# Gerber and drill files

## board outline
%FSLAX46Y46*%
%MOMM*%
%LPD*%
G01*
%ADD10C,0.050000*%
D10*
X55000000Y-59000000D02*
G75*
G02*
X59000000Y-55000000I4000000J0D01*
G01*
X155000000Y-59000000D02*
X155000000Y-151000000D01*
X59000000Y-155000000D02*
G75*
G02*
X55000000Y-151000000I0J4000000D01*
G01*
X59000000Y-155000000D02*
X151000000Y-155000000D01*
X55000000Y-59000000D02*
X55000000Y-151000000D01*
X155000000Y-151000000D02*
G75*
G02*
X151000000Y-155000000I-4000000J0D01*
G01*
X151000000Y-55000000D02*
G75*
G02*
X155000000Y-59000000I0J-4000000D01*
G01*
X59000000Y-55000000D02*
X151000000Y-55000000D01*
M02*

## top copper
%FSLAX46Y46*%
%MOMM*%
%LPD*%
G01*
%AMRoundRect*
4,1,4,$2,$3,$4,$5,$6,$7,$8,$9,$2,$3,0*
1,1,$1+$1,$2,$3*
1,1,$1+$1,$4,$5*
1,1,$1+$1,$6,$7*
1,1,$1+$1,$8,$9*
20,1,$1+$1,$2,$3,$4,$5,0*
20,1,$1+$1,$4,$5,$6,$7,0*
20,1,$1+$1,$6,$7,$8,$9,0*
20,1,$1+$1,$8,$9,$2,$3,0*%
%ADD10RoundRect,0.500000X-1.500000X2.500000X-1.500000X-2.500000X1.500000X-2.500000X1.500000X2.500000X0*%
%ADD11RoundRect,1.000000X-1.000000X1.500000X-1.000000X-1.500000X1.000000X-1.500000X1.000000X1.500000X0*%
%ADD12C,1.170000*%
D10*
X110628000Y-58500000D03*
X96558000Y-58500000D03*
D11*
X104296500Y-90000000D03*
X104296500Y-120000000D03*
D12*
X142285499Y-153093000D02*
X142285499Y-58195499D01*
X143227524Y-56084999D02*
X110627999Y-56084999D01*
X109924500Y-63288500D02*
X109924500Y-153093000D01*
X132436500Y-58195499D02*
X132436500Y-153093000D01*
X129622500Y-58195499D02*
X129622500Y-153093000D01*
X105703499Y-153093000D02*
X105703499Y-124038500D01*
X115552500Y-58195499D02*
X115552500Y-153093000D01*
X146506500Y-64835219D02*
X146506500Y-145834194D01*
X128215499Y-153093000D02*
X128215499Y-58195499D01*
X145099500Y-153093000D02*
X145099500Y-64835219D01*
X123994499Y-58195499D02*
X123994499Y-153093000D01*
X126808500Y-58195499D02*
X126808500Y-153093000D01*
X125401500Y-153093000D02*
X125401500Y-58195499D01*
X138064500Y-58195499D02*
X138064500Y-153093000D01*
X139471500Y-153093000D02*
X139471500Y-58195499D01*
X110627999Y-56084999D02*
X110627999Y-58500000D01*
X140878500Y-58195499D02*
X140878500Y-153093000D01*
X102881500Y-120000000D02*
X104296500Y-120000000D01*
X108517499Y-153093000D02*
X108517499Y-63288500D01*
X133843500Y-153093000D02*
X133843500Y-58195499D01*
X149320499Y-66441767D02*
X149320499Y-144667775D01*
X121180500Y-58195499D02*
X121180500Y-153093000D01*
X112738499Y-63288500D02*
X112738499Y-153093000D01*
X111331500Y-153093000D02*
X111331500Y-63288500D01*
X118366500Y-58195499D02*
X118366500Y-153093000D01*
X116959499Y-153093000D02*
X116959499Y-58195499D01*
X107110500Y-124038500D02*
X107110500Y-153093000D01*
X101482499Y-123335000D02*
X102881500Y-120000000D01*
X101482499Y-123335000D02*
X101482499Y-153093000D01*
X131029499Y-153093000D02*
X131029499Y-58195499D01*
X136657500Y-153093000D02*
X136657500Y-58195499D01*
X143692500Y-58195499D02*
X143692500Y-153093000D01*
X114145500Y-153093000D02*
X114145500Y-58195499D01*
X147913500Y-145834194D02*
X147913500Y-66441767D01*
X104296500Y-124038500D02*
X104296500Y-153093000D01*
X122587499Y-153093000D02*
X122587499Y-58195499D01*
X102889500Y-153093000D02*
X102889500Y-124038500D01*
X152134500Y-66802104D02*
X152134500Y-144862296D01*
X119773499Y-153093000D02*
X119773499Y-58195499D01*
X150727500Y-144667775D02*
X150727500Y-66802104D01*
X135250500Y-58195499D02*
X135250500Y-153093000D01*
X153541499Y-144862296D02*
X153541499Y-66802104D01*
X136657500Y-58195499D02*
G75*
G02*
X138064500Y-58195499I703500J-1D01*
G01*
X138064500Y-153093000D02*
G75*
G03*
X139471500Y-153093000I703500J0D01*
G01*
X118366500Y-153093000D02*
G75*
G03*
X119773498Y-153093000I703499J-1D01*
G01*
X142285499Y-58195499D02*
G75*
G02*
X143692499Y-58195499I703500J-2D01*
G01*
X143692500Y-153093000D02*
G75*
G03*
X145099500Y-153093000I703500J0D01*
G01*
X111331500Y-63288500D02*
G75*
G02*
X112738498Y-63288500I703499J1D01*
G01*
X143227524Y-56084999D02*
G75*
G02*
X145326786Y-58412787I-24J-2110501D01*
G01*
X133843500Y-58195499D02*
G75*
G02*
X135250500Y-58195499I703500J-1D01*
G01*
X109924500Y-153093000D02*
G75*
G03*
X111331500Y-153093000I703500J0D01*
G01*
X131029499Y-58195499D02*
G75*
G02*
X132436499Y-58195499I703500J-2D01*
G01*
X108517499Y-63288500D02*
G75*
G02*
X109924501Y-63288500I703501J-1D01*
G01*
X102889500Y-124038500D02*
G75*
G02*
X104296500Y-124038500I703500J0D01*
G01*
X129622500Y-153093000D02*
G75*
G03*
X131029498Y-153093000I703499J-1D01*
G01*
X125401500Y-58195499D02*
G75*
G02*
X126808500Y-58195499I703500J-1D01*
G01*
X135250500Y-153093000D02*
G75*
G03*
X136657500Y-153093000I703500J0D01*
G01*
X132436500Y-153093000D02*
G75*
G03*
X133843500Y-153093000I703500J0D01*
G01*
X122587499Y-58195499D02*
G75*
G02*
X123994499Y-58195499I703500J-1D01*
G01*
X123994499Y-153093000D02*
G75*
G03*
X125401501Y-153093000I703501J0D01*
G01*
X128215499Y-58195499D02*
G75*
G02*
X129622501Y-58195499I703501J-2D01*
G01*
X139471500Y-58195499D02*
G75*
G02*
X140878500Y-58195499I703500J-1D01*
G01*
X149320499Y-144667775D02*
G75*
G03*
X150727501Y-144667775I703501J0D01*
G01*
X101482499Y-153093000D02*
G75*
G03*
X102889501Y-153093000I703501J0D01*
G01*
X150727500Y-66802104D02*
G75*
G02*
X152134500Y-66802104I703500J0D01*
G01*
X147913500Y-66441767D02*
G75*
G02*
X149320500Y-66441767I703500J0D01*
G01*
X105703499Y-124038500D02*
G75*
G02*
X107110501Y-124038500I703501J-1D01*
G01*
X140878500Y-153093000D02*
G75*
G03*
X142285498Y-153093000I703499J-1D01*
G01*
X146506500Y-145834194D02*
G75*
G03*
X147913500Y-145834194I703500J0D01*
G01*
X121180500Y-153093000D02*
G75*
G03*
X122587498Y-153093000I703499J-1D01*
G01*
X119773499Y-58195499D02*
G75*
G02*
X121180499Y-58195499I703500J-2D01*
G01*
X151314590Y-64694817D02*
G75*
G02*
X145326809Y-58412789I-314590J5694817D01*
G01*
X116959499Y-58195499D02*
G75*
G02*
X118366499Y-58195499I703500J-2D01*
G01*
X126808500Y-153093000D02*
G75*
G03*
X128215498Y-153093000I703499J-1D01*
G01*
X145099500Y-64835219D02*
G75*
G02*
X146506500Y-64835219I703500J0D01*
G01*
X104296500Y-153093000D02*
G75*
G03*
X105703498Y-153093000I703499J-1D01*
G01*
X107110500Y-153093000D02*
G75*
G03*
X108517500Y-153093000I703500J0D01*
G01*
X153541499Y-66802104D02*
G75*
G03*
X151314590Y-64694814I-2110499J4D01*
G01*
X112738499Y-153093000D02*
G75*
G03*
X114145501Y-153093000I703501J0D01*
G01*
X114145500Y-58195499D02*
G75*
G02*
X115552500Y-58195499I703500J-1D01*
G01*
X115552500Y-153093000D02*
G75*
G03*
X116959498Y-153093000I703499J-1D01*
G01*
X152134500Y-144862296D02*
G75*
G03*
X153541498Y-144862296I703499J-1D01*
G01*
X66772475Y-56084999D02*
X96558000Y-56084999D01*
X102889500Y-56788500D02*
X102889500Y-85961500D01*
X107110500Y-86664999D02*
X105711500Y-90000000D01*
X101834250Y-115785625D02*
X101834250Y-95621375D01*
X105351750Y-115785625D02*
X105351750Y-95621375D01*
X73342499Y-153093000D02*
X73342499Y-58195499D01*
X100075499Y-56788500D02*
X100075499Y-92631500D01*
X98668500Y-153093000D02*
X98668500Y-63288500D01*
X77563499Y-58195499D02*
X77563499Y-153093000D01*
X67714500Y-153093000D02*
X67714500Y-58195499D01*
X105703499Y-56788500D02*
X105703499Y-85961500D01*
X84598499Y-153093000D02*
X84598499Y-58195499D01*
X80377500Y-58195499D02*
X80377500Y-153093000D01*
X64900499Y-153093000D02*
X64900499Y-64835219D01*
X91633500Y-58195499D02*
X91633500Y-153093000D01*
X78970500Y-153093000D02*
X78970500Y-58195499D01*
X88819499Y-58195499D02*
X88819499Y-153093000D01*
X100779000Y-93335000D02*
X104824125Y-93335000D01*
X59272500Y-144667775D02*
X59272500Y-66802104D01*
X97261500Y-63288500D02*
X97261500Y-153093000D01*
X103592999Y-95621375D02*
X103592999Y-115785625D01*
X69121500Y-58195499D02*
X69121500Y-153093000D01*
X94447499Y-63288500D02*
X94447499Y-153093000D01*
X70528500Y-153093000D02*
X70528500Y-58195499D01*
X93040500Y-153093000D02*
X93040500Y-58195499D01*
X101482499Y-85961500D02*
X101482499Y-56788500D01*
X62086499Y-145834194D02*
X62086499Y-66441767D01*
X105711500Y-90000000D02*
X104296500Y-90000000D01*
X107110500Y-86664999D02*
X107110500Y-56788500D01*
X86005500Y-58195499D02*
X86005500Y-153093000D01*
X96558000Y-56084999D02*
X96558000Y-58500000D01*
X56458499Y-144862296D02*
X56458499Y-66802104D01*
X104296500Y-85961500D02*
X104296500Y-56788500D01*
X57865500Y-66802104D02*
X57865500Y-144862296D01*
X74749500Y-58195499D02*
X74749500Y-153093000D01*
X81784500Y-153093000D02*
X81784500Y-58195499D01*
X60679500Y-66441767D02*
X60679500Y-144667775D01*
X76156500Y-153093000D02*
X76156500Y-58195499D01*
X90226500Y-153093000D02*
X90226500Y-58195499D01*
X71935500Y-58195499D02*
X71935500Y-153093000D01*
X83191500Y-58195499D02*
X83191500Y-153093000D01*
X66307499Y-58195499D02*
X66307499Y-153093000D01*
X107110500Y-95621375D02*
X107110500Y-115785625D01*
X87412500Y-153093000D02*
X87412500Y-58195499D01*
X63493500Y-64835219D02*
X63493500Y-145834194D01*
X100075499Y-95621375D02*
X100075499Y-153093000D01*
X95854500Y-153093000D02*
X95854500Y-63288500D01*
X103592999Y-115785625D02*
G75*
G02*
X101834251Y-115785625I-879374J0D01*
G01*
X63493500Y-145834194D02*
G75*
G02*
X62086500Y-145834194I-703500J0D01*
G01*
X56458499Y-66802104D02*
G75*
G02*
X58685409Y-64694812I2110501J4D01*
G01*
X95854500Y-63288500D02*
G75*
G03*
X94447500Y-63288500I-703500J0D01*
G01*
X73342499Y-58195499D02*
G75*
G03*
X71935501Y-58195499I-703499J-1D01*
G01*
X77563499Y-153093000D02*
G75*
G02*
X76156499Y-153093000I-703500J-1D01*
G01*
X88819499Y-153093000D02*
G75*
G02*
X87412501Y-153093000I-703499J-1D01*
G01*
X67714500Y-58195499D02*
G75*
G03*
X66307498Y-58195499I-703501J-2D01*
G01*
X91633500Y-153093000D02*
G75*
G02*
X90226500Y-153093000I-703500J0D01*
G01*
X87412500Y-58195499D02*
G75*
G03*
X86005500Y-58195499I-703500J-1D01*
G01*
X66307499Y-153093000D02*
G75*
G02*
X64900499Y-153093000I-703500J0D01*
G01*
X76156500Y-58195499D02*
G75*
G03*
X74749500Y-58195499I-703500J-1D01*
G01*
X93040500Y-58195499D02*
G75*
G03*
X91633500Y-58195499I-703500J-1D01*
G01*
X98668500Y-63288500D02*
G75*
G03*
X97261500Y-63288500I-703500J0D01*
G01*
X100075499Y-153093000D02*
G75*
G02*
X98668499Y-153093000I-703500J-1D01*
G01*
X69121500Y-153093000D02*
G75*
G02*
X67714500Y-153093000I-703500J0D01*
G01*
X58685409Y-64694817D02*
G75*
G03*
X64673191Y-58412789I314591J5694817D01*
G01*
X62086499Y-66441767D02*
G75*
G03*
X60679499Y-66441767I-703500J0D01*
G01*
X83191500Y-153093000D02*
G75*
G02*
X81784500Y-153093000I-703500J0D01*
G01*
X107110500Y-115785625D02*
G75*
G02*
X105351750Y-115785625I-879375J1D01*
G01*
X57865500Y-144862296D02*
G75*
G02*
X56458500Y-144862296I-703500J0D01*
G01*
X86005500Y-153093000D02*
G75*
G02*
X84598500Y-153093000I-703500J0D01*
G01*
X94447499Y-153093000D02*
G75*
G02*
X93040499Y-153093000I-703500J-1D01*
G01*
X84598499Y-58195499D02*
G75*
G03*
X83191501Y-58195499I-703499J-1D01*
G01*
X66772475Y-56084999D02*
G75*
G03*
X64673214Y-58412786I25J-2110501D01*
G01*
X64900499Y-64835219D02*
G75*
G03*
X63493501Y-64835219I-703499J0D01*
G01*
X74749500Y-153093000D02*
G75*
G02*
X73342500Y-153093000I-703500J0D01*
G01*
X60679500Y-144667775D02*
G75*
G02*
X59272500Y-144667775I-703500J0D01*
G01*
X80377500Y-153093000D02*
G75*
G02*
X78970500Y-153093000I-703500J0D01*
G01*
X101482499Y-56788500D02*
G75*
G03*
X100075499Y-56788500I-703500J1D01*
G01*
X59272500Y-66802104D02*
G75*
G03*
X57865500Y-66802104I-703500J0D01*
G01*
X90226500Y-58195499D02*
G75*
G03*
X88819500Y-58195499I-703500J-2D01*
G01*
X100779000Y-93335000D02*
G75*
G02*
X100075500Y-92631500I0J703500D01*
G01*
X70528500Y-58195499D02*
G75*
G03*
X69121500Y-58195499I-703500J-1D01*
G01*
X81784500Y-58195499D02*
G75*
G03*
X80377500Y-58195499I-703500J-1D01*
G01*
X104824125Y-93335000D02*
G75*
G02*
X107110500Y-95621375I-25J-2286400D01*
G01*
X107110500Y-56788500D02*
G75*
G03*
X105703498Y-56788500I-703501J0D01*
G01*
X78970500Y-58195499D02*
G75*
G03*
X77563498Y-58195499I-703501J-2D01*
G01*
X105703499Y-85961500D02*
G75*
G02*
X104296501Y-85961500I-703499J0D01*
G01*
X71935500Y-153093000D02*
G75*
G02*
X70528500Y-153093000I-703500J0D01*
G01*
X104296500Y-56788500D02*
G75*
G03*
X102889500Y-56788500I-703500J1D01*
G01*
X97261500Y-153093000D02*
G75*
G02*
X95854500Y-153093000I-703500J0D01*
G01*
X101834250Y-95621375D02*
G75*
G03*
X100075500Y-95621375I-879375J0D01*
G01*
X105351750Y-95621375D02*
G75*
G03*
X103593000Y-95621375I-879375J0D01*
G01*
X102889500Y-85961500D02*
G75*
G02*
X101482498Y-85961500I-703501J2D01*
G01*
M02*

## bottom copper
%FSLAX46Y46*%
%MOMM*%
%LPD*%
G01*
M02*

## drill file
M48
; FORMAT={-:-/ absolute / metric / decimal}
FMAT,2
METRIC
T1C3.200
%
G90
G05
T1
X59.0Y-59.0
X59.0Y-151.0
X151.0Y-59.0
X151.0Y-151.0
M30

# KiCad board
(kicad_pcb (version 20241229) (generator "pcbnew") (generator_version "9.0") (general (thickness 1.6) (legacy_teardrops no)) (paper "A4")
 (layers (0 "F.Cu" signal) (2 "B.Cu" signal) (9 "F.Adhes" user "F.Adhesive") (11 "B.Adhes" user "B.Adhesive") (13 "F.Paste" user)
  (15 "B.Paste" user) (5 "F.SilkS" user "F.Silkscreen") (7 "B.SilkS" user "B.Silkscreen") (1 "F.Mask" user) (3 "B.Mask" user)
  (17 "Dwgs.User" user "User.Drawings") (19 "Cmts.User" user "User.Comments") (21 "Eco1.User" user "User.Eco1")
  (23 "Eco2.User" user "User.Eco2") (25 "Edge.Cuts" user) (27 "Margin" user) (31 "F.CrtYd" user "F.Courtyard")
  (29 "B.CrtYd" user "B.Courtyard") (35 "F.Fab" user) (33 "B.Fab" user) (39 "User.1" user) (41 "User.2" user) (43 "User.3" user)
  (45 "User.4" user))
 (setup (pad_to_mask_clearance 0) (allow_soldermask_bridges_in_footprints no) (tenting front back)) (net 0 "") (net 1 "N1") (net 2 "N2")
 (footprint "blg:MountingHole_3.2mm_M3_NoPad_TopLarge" (layer "F.Cu") (at 151 59)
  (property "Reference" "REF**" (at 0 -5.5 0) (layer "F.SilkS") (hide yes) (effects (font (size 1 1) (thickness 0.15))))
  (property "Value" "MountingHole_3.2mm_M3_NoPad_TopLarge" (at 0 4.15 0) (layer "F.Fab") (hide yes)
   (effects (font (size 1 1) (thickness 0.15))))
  (pad "" np_thru_hole circle (at 0 0) (size 7.6 7.6) (drill 3.2) (layers) (zone_connect 2)))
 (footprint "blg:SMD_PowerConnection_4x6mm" (layer "F.Cu") (at 110.628 58.5 -90)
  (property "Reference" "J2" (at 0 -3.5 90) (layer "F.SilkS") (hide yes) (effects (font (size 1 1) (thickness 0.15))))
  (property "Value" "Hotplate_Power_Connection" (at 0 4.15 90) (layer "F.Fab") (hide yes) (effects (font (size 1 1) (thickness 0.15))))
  (pad "1" smd roundrect (at 0 0 270) (size 6 4) (layers "F.Cu" "F.Mask" "F.Paste") (roundrect_rratio 0.125) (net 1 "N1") (zone_connect 2)))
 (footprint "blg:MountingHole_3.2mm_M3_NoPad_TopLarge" (layer "F.Cu") (at 59 151)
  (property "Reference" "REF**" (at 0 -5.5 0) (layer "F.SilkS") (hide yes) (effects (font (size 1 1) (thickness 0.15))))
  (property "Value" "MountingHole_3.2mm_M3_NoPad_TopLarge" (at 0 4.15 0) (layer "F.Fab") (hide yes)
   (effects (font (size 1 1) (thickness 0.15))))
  (pad "" np_thru_hole circle (at 0 0) (size 7.6 7.6) (drill 3.2) (layers) (zone_connect 2)))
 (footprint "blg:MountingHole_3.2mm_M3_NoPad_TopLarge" (layer "F.Cu") (at 151 151)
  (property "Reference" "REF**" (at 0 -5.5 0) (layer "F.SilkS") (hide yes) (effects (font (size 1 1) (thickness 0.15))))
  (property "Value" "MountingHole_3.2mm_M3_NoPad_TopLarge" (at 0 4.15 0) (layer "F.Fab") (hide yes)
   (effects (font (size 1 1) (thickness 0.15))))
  (pad "" np_thru_hole circle (at 0 0) (size 7.6 7.6) (drill 3.2) (layers) (zone_connect 2)))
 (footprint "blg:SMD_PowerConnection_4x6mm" (layer "F.Cu") (at 96.558 58.5 -90)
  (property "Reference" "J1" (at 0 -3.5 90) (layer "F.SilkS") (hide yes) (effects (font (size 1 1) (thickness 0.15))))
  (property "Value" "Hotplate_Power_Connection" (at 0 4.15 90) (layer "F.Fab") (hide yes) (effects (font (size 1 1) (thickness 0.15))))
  (pad "1" smd roundrect (at 0 0 270) (size 6 4) (layers "F.Cu" "F.Mask" "F.Paste") (roundrect_rratio 0.125) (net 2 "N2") (zone_connect 2)))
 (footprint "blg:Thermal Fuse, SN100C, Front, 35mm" (layer "F.Cu") (at 104.2965 105 -90)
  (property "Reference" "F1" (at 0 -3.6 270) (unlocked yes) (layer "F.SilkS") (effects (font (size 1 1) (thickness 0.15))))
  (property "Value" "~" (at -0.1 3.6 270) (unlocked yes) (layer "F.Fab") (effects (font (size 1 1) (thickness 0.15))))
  (pad "1" smd roundrect (at -15 0 270) (size 5 4) (layers "F.Cu" "F.Mask") (roundrect_rratio 0.25) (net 2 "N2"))
  (pad "2" smd roundrect (at 15 0 270) (size 5 4) (layers "F.Cu" "F.Mask") (roundrect_rratio 0.25) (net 1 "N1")))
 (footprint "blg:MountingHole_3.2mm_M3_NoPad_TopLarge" (layer "F.Cu") (at 59 59)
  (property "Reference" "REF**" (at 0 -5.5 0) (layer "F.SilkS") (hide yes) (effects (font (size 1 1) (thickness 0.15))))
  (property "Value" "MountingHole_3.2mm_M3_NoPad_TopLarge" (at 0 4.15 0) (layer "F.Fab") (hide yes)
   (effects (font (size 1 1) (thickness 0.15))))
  (pad "" np_thru_hole circle (at 0 0) (size 7.6 7.6) (drill 3.2) (layers) (zone_connect 2)))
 (gr_arc (start 55 59) (mid 56.171573 56.171573) (end 59 55) (stroke (width 0.05) (type solid)) (layer "Edge.Cuts"))
 (gr_line (start 155 59) (end 155 151) (stroke (width 0.05) (type default)) (layer "Edge.Cuts"))
 (gr_arc (start 59 155) (mid 56.171573 153.828427) (end 55 151) (stroke (width 0.05) (type solid)) (layer "Edge.Cuts"))
 (gr_line (start 59 155) (end 151 155) (stroke (width 0.05) (type default)) (layer "Edge.Cuts"))
 (gr_line (start 55 59) (end 55 151) (stroke (width 0.05) (type default)) (layer "Edge.Cuts"))
 (gr_arc (start 155 151) (mid 153.828427 153.828427) (end 151 155) (stroke (width 0.05) (type solid)) (layer "Edge.Cuts"))
 (gr_arc (start 151 55) (mid 153.828427 56.171573) (end 155 59) (stroke (width 0.05) (type solid)) (layer "Edge.Cuts"))
 (gr_line (start 59 55) (end 151 55) (stroke (width 0.05) (type default)) (layer "Edge.Cuts"))
 (segment (start 142.285499 153.093) (end 142.285499 58.195499) (width 1.17) (layer "F.Cu") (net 1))
 (segment (start 143.227524 56.084999) (end 110.627999 56.084999) (width 1.17) (layer "F.Cu") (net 1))
 (segment (start 109.9245 63.2885) (end 109.9245 153.093) (width 1.17) (layer "F.Cu") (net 1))
 (segment (start 132.4365 58.195499) (end 132.4365 153.093) (width 1.17) (layer "F.Cu") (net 1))
 (segment (start 129.6225 58.195499) (end 129.6225 153.093) (width 1.17) (layer "F.Cu") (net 1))
 (segment (start 105.703499 153.093) (end 105.703499 124.0385) (width 1.17) (layer "F.Cu") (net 1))
 (segment (start 115.5525 58.195499) (end 115.5525 153.093) (width 1.17) (layer "F.Cu") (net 1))
 (segment (start 146.5065 64.835219) (end 146.5065 145.834194) (width 1.17) (layer "F.Cu") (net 1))
 (segment (start 128.215499 153.093) (end 128.215499 58.195499) (width 1.17) (layer "F.Cu") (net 1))
 (segment (start 145.0995 153.093) (end 145.0995 64.835219) (width 1.17) (layer "F.Cu") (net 1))
 (segment (start 123.994499 58.195499) (end 123.994499 153.093) (width 1.17) (layer "F.Cu") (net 1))
 (segment (start 126.8085 58.195499) (end 126.8085 153.093) (width 1.17) (layer "F.Cu") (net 1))
 (segment (start 125.4015 153.093) (end 125.4015 58.195499) (width 1.17) (layer "F.Cu") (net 1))
 (segment (start 138.0645 58.195499) (end 138.0645 153.093) (width 1.17) (layer "F.Cu") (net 1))
 (segment (start 139.4715 153.093) (end 139.4715 58.195499) (width 1.17) (layer "F.Cu") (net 1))
 (segment (start 110.627999 56.084999) (end 110.627999 58.5) (width 1.17) (layer "F.Cu") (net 1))
 (segment (start 140.8785 58.195499) (end 140.8785 153.093) (width 1.17) (layer "F.Cu") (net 1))
 (segment (start 102.8815 120) (end 104.2965 120) (width 1.17) (layer "F.Cu") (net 1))
 (segment (start 108.517499 153.093) (end 108.517499 63.2885) (width 1.17) (layer "F.Cu") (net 1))
 (segment (start 133.8435 153.093) (end 133.8435 58.195499) (width 1.17) (layer "F.Cu") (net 1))
 (segment (start 149.320499 66.441767) (end 149.320499 144.667775) (width 1.17) (layer "F.Cu") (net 1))
 (segment (start 121.1805 58.195499) (end 121.1805 153.093) (width 1.17) (layer "F.Cu") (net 1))
 (segment (start 112.738499 63.2885) (end 112.738499 153.093) (width 1.17) (layer "F.Cu") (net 1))
 (segment (start 111.3315 153.093) (end 111.3315 63.2885) (width 1.17) (layer "F.Cu") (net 1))
 (segment (start 118.3665 58.195499) (end 118.3665 153.093) (width 1.17) (layer "F.Cu") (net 1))
 (segment (start 116.959499 153.093) (end 116.959499 58.195499) (width 1.17) (layer "F.Cu") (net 1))
 (segment (start 107.1105 124.0385) (end 107.1105 153.093) (width 1.17) (layer "F.Cu") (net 1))
 (segment (start 101.482499 123.335) (end 102.8815 120) (width 1.17) (layer "F.Cu") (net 1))
 (segment (start 101.482499 123.335) (end 101.482499 153.093) (width 1.17) (layer "F.Cu") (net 1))
 (segment (start 131.029499 153.093) (end 131.029499 58.195499) (width 1.17) (layer "F.Cu") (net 1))
 (segment (start 136.6575 153.093) (end 136.6575 58.195499) (width 1.17) (layer "F.Cu") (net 1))
 (segment (start 143.6925 58.195499) (end 143.6925 153.093) (width 1.17) (layer "F.Cu") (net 1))
 (segment (start 114.1455 153.093) (end 114.1455 58.195499) (width 1.17) (layer "F.Cu") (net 1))
 (segment (start 147.9135 145.834194) (end 147.9135 66.441767) (width 1.17) (layer "F.Cu") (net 1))
 (segment (start 104.2965 124.0385) (end 104.2965 153.093) (width 1.17) (layer "F.Cu") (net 1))
 (segment (start 122.587499 153.093) (end 122.587499 58.195499) (width 1.17) (layer "F.Cu") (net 1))
 (segment (start 102.8895 153.093) (end 102.8895 124.0385) (width 1.17) (layer "F.Cu") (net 1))
 (segment (start 152.1345 66.802104) (end 152.1345 144.862296) (width 1.17) (layer "F.Cu") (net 1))
 (segment (start 119.773499 153.093) (end 119.773499 58.195499) (width 1.17) (layer "F.Cu") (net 1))
 (segment (start 150.7275 144.667775) (end 150.7275 66.802104) (width 1.17) (layer "F.Cu") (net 1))
 (segment (start 135.2505 58.195499) (end 135.2505 153.093) (width 1.17) (layer "F.Cu") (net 1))
 (segment (start 153.541499 144.862296) (end 153.541499 66.802104) (width 1.17) (layer "F.Cu") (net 1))
 (arc (start 136.6575 58.195499) (mid 137.361 57.492) (end 138.0645 58.195499) (width 1.17) (layer "F.Cu") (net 1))
 (arc (start 138.0645 153.093) (mid 138.768 153.7965) (end 139.4715 153.093) (width 1.17) (layer "F.Cu") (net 1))
 (arc (start 118.3665 153.093) (mid 119.07 153.7965) (end 119.773499 153.093) (width 1.17) (layer "F.Cu") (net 1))
 (arc (start 142.285499 58.195499) (mid 142.989 57.492) (end 143.6925 58.195499) (width 1.17) (layer "F.Cu") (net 1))
 (arc (start 143.6925 153.093) (mid 144.396 153.7965) (end 145.0995 153.093) (width 1.17) (layer "F.Cu") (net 1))
 (arc (start 111.3315 63.2885) (mid 112.035 62.585) (end 112.738499 63.2885) (width 1.17) (layer "F.Cu") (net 1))
 (arc (start 143.227524 56.084999) (mid 144.794814 56.78206) (end 145.326809 58.412789) (width 1.17) (layer "F.Cu") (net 1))
 (arc (start 133.8435 58.195499) (mid 134.547 57.492) (end 135.2505 58.195499) (width 1.17) (layer "F.Cu") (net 1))
 (arc (start 109.9245 153.093) (mid 110.627999 153.7965) (end 111.3315 153.093) (width 1.17) (layer "F.Cu") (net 1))
 (arc (start 131.029499 58.195499) (mid 131.732999 57.492) (end 132.4365 58.195499) (width 1.17) (layer "F.Cu") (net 1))
 (arc (start 108.517499 63.2885) (mid 109.221 62.585) (end 109.9245 63.2885) (width 1.17) (layer "F.Cu") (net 1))
 (arc (start 102.8895 124.0385) (mid 103.592999 123.335) (end 104.2965 124.0385) (width 1.17) (layer "F.Cu") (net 1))
 (arc (start 129.6225 153.093) (mid 130.326 153.7965) (end 131.029499 153.093) (width 1.17) (layer "F.Cu") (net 1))
 (arc (start 125.4015 58.195499) (mid 126.104999 57.492) (end 126.8085 58.195499) (width 1.17) (layer "F.Cu") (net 1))
 (arc (start 135.2505 153.093) (mid 135.953999 153.7965) (end 136.6575 153.093) (width 1.17) (layer "F.Cu") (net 1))
 (arc (start 132.4365 153.093) (mid 133.139999 153.7965) (end 133.8435 153.093) (width 1.17) (layer "F.Cu") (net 1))
 (arc (start 122.587499 58.195499) (mid 123.291 57.492) (end 123.994499 58.195499) (width 1.17) (layer "F.Cu") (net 1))
 (arc (start 123.994499 153.093) (mid 124.698 153.7965) (end 125.4015 153.093) (width 1.17) (layer "F.Cu") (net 1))
 (arc (start 128.215499 58.195499) (mid 128.919 57.492) (end 129.6225 58.195499) (width 1.17) (layer "F.Cu") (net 1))
 (arc (start 139.4715 58.195499) (mid 140.174999 57.492) (end 140.8785 58.195499) (width 1.17) (layer "F.Cu") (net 1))
 (arc (start 149.320499 144.667775) (mid 150.024 145.371275) (end 150.7275 144.667775) (width 1.17) (layer "F.Cu") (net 1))
 (arc (start 101.482499 153.093) (mid 102.186 153.7965) (end 102.8895 153.093) (width 1.17) (layer "F.Cu") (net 1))
 (arc (start 150.7275 66.802104) (mid 151.430999 66.098604) (end 152.1345 66.802104) (width 1.17) (layer "F.Cu") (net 1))
 (arc (start 147.9135 66.441767) (mid 148.617 65.738267) (end 149.320499 66.441767) (width 1.17) (layer "F.Cu") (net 1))
 (arc (start 105.703499 124.0385) (mid 106.407 123.335) (end 107.1105 124.0385) (width 1.17) (layer "F.Cu") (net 1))
 (arc (start 140.8785 153.093) (mid 141.582 153.7965) (end 142.285499 153.093) (width 1.17) (layer "F.Cu") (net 1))
 (arc (start 146.5065 145.834194) (mid 147.209999 146.537694) (end 147.9135 145.834194) (width 1.17) (layer "F.Cu") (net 1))
 (arc (start 121.1805 153.093) (mid 121.883999 153.7965) (end 122.587499 153.093) (width 1.17) (layer "F.Cu") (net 1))
 (arc (start 119.773499 58.195499) (mid 120.477 57.492) (end 121.1805 58.195499) (width 1.17) (layer "F.Cu") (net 1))
 (arc (start 151.31459 64.694817) (mid 146.871486 62.935135) (end 145.326809 58.412789) (width 1.17) (layer "F.Cu") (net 1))
 (arc (start 116.959499 58.195499) (mid 117.663 57.492) (end 118.3665 58.195499) (width 1.17) (layer "F.Cu") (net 1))
 (arc (start 126.8085 153.093) (mid 127.511999 153.7965) (end 128.215499 153.093) (width 1.17) (layer "F.Cu") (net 1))
 (arc (start 145.0995 64.835219) (mid 145.803 64.131719) (end 146.5065 64.835219) (width 1.17) (layer "F.Cu") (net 1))
 (arc (start 104.2965 153.093) (mid 105 153.7965) (end 105.703499 153.093) (width 1.17) (layer "F.Cu") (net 1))
 (arc (start 107.1105 153.093) (mid 107.814 153.7965) (end 108.5175 153.093) (width 1.17) (layer "F.Cu") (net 1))
 (arc (start 153.541499 66.802104) (mid 152.969318 65.357186) (end 151.31459 64.694817) (width 1.17) (layer "F.Cu") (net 1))
 (arc (start 112.738499 153.093) (mid 113.442 153.7965) (end 114.1455 153.093) (width 1.17) (layer "F.Cu") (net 1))
 (arc (start 114.1455 58.195499) (mid 114.848999 57.492) (end 115.5525 58.195499) (width 1.17) (layer "F.Cu") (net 1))
 (arc (start 115.5525 153.093) (mid 116.256 153.7965) (end 116.959499 153.093) (width 1.17) (layer "F.Cu") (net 1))
 (arc (start 152.1345 144.862296) (mid 152.838 145.565796) (end 153.541499 144.862296) (width 1.17) (layer "F.Cu") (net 1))
 (segment (start 66.772475 56.084999) (end 96.558 56.084999) (width 1.17) (layer "F.Cu") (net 2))
 (segment (start 102.8895 56.7885) (end 102.8895 85.9615) (width 1.17) (layer "F.Cu") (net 2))
 (segment (start 107.1105 86.664999) (end 105.7115 90) (width 1.17) (layer "F.Cu") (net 2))
 (segment (start 101.83425 115.785625) (end 101.83425 95.621375) (width 1.17) (layer "F.Cu") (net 2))
 (segment (start 105.35175 115.785625) (end 105.35175 95.621375) (width 1.17) (layer "F.Cu") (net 2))
 (segment (start 73.342499 153.093) (end 73.342499 58.195499) (width 1.17) (layer "F.Cu") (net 2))
 (segment (start 100.075499 56.7885) (end 100.075499 92.6315) (width 1.17) (layer "F.Cu") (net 2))
 (segment (start 98.6685 153.093) (end 98.6685 63.2885) (width 1.17) (layer "F.Cu") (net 2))
 (segment (start 77.563499 58.195499) (end 77.563499 153.093) (width 1.17) (layer "F.Cu") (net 2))
 (segment (start 67.7145 153.093) (end 67.7145 58.195499) (width 1.17) (layer "F.Cu") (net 2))
 (segment (start 105.703499 56.7885) (end 105.703499 85.9615) (width 1.17) (layer "F.Cu") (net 2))
 (segment (start 84.598499 153.093) (end 84.598499 58.195499) (width 1.17) (layer "F.Cu") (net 2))
 (segment (start 80.3775 58.195499) (end 80.3775 153.093) (width 1.17) (layer "F.Cu") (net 2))
 (segment (start 64.900499 153.093) (end 64.900499 64.835219) (width 1.17) (layer "F.Cu") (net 2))
 (segment (start 91.6335 58.195499) (end 91.6335 153.093) (width 1.17) (layer "F.Cu") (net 2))
 (segment (start 78.9705 153.093) (end 78.9705 58.195499) (width 1.17) (layer "F.Cu") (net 2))
 (segment (start 88.819499 58.195499) (end 88.819499 153.093) (width 1.17) (layer "F.Cu") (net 2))
 (segment (start 100.779 93.335) (end 104.824125 93.335) (width 1.17) (layer "F.Cu") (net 2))
 (segment (start 59.2725 144.667775) (end 59.2725 66.802104) (width 1.17) (layer "F.Cu") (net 2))
 (segment (start 97.2615 63.2885) (end 97.2615 153.093) (width 1.17) (layer "F.Cu") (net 2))
 (segment (start 103.592999 95.621375) (end 103.592999 115.785625) (width 1.17) (layer "F.Cu") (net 2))
 (segment (start 69.1215 58.195499) (end 69.1215 153.093) (width 1.17) (layer "F.Cu") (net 2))
 (segment (start 94.447499 63.2885) (end 94.447499 153.093) (width 1.17) (layer "F.Cu") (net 2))
 (segment (start 70.5285 153.093) (end 70.5285 58.195499) (width 1.17) (layer "F.Cu") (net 2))
 (segment (start 93.0405 153.093) (end 93.0405 58.195499) (width 1.17) (layer "F.Cu") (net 2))
 (segment (start 101.482499 85.9615) (end 101.482499 56.7885) (width 1.17) (layer "F.Cu") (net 2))
 (segment (start 62.086499 145.834194) (end 62.086499 66.441767) (width 1.17) (layer "F.Cu") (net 2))
 (segment (start 105.7115 90) (end 104.2965 90) (width 1.17) (layer "F.Cu") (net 2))
 (segment (start 107.1105 86.664999) (end 107.1105 56.7885) (width 1.17) (layer "F.Cu") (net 2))
 (segment (start 86.0055 58.195499) (end 86.0055 153.093) (width 1.17) (layer "F.Cu") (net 2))
 (segment (start 96.558 56.084999) (end 96.558 58.5) (width 1.17) (layer "F.Cu") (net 2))
 (segment (start 56.458499 144.862296) (end 56.458499 66.802104) (width 1.17) (layer "F.Cu") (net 2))
 (segment (start 104.2965 85.9615) (end 104.2965 56.7885) (width 1.17) (layer "F.Cu") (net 2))
 (segment (start 57.8655 66.802104) (end 57.8655 144.862296) (width 1.17) (layer "F.Cu") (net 2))
 (segment (start 74.7495 58.195499) (end 74.7495 153.093) (width 1.17) (layer "F.Cu") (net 2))
 (segment (start 81.7845 153.093) (end 81.7845 58.195499) (width 1.17) (layer "F.Cu") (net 2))
 (segment (start 60.6795 66.441767) (end 60.6795 144.667775) (width 1.17) (layer "F.Cu") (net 2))
 (segment (start 76.1565 153.093) (end 76.1565 58.195499) (width 1.17) (layer "F.Cu") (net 2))
 (segment (start 90.2265 153.093) (end 90.2265 58.195499) (width 1.17) (layer "F.Cu") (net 2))
 (segment (start 71.9355 58.195499) (end 71.9355 153.093) (width 1.17) (layer "F.Cu") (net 2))
 (segment (start 83.1915 58.195499) (end 83.1915 153.093) (width 1.17) (layer "F.Cu") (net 2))
 (segment (start 66.307499 58.195499) (end 66.307499 153.093) (width 1.17) (layer "F.Cu") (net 2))
 (segment (start 107.1105 95.621375) (end 107.1105 115.785625) (width 1.17) (layer "F.Cu") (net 2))
 (segment (start 87.4125 153.093) (end 87.4125 58.195499) (width 1.17) (layer "F.Cu") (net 2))
 (segment (start 63.4935 64.835219) (end 63.4935 145.834194) (width 1.17) (layer "F.Cu") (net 2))
 (segment (start 100.075499 95.621375) (end 100.075499 153.093) (width 1.17) (layer "F.Cu") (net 2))
 (segment (start 95.8545 153.093) (end 95.8545 63.2885) (width 1.17) (layer "F.Cu") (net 2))
 (arc (start 103.592999 115.785625) (mid 102.713625 116.664999) (end 101.83425 115.785625) (width 1.17) (layer "F.Cu") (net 2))
 (arc (start 63.4935 145.834194) (mid 62.79 146.537694) (end 62.086499 145.834194) (width 1.17) (layer "F.Cu") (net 2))
 (arc (start 56.458499 66.802104) (mid 57.030681 65.357186) (end 58.685409 64.694817) (width 1.17) (layer "F.Cu") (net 2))
 (arc (start 95.8545 63.2885) (mid 95.151 62.585) (end 94.447499 63.2885) (width 1.17) (layer "F.Cu") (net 2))
 (arc (start 73.342499 58.195499) (mid 72.639 57.492) (end 71.9355 58.195499) (width 1.17) (layer "F.Cu") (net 2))
 (arc (start 77.563499 153.093) (mid 76.86 153.7965) (end 76.1565 153.093) (width 1.17) (layer "F.Cu") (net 2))
 (arc (start 88.819499 153.093) (mid 88.116 153.7965) (end 87.4125 153.093) (width 1.17) (layer "F.Cu") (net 2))
 (arc (start 67.7145 58.195499) (mid 67.010999 57.492) (end 66.307499 58.195499) (width 1.17) (layer "F.Cu") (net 2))
 (arc (start 91.6335 153.093) (mid 90.93 153.7965) (end 90.2265 153.093) (width 1.17) (layer "F.Cu") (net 2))
 (arc (start 87.4125 58.195499) (mid 86.708999 57.492) (end 86.0055 58.195499) (width 1.17) (layer "F.Cu") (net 2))
 (arc (start 66.307499 153.093) (mid 65.604 153.7965) (end 64.900499 153.093) (width 1.17) (layer "F.Cu") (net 2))
 (arc (start 76.1565 58.195499) (mid 75.452999 57.492) (end 74.7495 58.195499) (width 1.17) (layer "F.Cu") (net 2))
 (arc (start 93.0405 58.195499) (mid 92.337 57.492) (end 91.6335 58.195499) (width 1.17) (layer "F.Cu") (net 2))
 (arc (start 98.6685 63.2885) (mid 97.965 62.585) (end 97.2615 63.2885) (width 1.17) (layer "F.Cu") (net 2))
 (arc (start 100.075499 153.093) (mid 99.372 153.7965) (end 98.6685 153.093) (width 1.17) (layer "F.Cu") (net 2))
 (arc (start 69.1215 153.093) (mid 68.417999 153.7965) (end 67.7145 153.093) (width 1.17) (layer "F.Cu") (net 2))
 (arc (start 58.685409 64.694817) (mid 63.128513 62.935135) (end 64.67319 58.412789) (width 1.17) (layer "F.Cu") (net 2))
 (arc (start 62.086499 66.441767) (mid 61.383 65.738267) (end 60.6795 66.441767) (width 1.17) (layer "F.Cu") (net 2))
 (arc (start 83.1915 153.093) (mid 82.487999 153.7965) (end 81.7845 153.093) (width 1.17) (layer "F.Cu") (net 2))
 (arc (start 107.1105 115.785625) (mid 106.231124 116.664999) (end 105.35175 115.785625) (width 1.17) (layer "F.Cu") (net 2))
 (arc (start 57.8655 144.862296) (mid 57.162 145.565796) (end 56.458499 144.862296) (width 1.17) (layer "F.Cu") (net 2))
 (arc (start 86.0055 153.093) (mid 85.302 153.7965) (end 84.598499 153.093) (width 1.17) (layer "F.Cu") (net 2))
 (arc (start 94.447499 153.093) (mid 93.744 153.7965) (end 93.0405 153.093) (width 1.17) (layer "F.Cu") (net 2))
 (arc (start 84.598499 58.195499) (mid 83.895 57.492) (end 83.1915 58.195499) (width 1.17) (layer "F.Cu") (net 2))
 (arc (start 66.772475 56.084999) (mid 65.205185 56.78206) (end 64.67319 58.412789) (width 1.17) (layer "F.Cu") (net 2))
 (arc (start 64.900499 64.835219) (mid 64.196999 64.131719) (end 63.4935 64.835219) (width 1.17) (layer "F.Cu") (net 2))
 (arc (start 74.7495 153.093) (mid 74.046 153.7965) (end 73.342499 153.093) (width 1.17) (layer "F.Cu") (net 2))
 (arc (start 60.6795 144.667775) (mid 59.975999 145.371275) (end 59.2725 144.667775) (width 1.17) (layer "F.Cu") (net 2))
 (arc (start 80.3775 153.093) (mid 79.673999 153.7965) (end 78.9705 153.093) (width 1.17) (layer "F.Cu") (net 2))
 (arc (start 101.482499 56.7885) (mid 100.779 56.084999) (end 100.075499 56.7885) (width 1.17) (layer "F.Cu") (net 2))
 (arc (start 59.2725 66.802104) (mid 58.568999 66.098604) (end 57.8655 66.802104) (width 1.17) (layer "F.Cu") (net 2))
 (arc (start 90.2265 58.195499) (mid 89.523 57.492) (end 88.819499 58.195499) (width 1.17) (layer "F.Cu") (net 2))
 (arc (start 100.779 93.335) (mid 100.28155 93.128949) (end 100.075499 92.6315) (width 1.17) (layer "F.Cu") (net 2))
 (arc (start 70.5285 58.195499) (mid 69.825 57.492) (end 69.1215 58.195499) (width 1.17) (layer "F.Cu") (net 2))
 (arc (start 81.7845 58.195499) (mid 81.081 57.492) (end 80.3775 58.195499) (width 1.17) (layer "F.Cu") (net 2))
 (arc (start 104.824125 93.335) (mid 106.440836 94.004663) (end 107.1105 95.621375) (width 1.17) (layer "F.Cu") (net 2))
 (arc (start 107.1105 56.7885) (mid 106.407 56.084999) (end 105.703499 56.7885) (width 1.17) (layer "F.Cu") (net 2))
 (arc (start 78.9705 58.195499) (mid 78.267 57.492) (end 77.563499 58.195499) (width 1.17) (layer "F.Cu") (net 2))
 (arc (start 105.703499 85.9615) (mid 105 86.664999) (end 104.2965 85.9615) (width 1.17) (layer "F.Cu") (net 2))
 (arc (start 71.9355 153.093) (mid 71.232 153.7965) (end 70.5285 153.093) (width 1.17) (layer "F.Cu") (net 2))
 (arc (start 104.2965 56.7885) (mid 103.592999 56.084999) (end 102.8895 56.7885) (width 1.17) (layer "F.Cu") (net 2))
 (arc (start 97.2615 153.093) (mid 96.558 153.7965) (end 95.8545 153.093) (width 1.17) (layer "F.Cu") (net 2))
 (arc (start 101.83425 95.621375) (mid 100.954875 94.741999) (end 100.075499 95.621375) (width 1.17) (layer "F.Cu") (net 2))
 (arc (start 105.35175 95.621375) (mid 104.472374 94.741999) (end 103.592999 95.621375) (width 1.17) (layer "F.Cu") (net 2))
 (arc (start 102.8895 85.9615) (mid 102.186 86.664999) (end 101.482499 85.9615) (width 1.17) (layer "F.Cu") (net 2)))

